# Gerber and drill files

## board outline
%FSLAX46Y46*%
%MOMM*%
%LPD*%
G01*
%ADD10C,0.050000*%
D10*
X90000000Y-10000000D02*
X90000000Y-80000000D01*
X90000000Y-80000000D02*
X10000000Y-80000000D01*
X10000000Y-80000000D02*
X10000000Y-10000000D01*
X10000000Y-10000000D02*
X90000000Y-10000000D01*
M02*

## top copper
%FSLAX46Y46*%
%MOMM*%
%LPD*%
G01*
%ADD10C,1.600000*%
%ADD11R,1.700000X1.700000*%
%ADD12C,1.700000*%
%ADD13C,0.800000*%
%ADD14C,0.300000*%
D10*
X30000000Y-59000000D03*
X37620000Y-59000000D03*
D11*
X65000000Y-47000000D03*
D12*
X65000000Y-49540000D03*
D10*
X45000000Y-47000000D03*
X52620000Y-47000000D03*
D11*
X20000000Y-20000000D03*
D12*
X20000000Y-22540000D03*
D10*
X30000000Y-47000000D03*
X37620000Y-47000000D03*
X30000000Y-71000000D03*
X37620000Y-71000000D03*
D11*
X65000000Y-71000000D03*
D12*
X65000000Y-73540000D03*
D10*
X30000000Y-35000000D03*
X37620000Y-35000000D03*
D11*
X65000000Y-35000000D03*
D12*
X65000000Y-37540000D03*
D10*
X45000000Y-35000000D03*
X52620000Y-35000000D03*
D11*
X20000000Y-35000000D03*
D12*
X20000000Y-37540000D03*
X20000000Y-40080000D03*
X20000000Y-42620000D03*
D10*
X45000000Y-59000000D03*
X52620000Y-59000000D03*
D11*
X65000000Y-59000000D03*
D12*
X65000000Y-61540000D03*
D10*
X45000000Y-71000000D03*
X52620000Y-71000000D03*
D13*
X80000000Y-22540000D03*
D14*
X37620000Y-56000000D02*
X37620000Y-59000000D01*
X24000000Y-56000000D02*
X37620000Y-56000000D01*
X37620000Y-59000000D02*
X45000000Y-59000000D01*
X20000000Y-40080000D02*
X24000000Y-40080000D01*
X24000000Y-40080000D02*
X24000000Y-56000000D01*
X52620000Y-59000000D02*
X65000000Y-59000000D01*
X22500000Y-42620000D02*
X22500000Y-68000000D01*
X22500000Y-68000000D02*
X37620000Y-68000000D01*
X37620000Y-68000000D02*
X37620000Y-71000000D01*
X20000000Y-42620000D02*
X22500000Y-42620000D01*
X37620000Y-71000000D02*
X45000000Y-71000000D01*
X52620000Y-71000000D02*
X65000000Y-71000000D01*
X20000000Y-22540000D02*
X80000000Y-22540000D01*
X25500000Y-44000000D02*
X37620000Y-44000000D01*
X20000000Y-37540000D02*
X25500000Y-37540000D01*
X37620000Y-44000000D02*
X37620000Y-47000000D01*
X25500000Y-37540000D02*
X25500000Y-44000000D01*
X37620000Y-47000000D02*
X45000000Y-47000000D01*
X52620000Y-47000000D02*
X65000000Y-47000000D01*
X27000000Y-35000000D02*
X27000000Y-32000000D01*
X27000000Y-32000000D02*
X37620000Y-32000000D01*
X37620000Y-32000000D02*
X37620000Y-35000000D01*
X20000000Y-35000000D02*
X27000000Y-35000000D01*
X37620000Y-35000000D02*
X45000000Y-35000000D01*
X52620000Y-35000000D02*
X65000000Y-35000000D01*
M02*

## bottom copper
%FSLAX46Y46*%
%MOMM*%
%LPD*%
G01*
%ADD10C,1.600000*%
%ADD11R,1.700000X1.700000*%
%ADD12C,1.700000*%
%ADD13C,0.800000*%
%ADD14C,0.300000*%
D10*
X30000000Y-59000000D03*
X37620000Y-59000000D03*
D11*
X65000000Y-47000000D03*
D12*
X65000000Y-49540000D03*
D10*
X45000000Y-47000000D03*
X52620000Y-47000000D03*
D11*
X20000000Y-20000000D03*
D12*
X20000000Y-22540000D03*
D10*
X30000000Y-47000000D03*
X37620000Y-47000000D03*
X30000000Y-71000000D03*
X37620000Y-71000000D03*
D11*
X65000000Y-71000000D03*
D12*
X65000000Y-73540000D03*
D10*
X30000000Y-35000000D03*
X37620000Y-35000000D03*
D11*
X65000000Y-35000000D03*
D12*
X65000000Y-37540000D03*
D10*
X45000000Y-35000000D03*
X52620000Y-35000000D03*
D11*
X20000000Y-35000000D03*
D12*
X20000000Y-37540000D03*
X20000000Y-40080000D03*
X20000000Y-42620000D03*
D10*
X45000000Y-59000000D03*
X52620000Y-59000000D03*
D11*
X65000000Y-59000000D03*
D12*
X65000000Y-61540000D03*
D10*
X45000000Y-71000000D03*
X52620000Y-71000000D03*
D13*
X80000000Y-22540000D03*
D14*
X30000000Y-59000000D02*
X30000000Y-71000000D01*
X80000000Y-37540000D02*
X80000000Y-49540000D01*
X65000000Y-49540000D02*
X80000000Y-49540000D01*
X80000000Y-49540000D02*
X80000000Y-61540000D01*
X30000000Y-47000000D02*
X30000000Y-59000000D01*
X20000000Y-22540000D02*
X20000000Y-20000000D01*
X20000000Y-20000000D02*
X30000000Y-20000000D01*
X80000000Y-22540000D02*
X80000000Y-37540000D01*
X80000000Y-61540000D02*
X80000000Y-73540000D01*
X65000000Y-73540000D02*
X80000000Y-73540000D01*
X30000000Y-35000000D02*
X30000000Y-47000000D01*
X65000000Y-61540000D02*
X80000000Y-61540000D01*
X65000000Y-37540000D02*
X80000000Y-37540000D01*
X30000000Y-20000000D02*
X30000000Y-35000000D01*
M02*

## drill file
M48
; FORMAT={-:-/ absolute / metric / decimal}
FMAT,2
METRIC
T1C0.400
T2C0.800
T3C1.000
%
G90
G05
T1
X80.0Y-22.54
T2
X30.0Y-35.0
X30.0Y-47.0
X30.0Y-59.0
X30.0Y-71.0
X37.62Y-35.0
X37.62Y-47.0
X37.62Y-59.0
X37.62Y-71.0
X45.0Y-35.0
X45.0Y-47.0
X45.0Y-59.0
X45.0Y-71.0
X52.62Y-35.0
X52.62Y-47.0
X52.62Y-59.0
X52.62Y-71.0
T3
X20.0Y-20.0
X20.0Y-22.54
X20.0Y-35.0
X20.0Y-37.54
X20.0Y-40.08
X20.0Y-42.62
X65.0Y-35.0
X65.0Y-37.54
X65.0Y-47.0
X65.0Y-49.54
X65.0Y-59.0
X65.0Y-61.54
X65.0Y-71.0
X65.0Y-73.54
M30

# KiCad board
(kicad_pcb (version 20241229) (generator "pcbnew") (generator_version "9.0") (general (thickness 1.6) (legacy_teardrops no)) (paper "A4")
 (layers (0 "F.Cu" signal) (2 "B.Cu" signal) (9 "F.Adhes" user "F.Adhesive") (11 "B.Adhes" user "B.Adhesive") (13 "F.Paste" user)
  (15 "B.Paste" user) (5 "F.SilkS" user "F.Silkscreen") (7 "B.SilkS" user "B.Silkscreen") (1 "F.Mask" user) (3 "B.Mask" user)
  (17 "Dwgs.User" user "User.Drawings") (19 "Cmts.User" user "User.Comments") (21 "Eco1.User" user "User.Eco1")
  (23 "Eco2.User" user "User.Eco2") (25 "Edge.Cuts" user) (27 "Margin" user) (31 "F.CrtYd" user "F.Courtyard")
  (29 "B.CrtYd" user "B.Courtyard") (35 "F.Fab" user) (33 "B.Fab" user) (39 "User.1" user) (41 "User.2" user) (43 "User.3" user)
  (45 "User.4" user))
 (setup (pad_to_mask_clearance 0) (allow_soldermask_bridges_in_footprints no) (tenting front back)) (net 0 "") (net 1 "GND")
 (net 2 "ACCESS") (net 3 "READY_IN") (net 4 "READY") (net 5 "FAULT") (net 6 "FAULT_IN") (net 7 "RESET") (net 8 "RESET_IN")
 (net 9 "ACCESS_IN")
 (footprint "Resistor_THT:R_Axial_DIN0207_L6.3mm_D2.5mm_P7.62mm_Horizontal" (layer "F.Cu") (at 30 59)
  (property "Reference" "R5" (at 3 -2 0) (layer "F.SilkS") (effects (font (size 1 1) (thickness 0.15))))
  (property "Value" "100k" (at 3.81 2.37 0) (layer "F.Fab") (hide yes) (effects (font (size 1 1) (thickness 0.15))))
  (pad "1" thru_hole circle (at 0 0) (size 1.6 1.6) (drill 0.8) (layers "*.Cu" "*.Mask") (remove_unused_layers no) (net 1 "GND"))
  (pad "2" thru_hole circle (at 7.62 0) (size 1.6 1.6) (drill 0.8) (layers "*.Cu" "*.Mask") (remove_unused_layers no) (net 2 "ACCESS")))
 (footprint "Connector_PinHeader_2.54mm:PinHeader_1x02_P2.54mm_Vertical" (layer "F.Cu") (at 65 47)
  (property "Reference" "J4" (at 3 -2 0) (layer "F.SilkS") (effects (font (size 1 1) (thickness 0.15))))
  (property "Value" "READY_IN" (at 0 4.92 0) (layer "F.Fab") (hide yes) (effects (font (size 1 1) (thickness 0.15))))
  (pad "1" thru_hole rect (at 0 0) (size 1.7 1.7) (drill 1) (layers "*.Cu" "*.Mask") (remove_unused_layers no) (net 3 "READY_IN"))
  (pad "2" thru_hole circle (at 0 2.54) (size 1.7 1.7) (drill 1) (layers "*.Cu" "*.Mask") (remove_unused_layers no) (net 1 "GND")))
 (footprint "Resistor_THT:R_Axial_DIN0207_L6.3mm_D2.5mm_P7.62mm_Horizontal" (layer "F.Cu") (at 45 47)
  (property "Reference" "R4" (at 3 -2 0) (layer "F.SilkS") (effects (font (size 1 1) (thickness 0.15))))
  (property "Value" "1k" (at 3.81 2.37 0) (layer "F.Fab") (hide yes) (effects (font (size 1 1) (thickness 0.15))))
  (pad "1" thru_hole circle (at 0 0) (size 1.6 1.6) (drill 0.8) (layers "*.Cu" "*.Mask") (remove_unused_layers no) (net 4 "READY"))
  (pad "2" thru_hole circle (at 7.62 0) (size 1.6 1.6) (drill 0.8) (layers "*.Cu" "*.Mask") (remove_unused_layers no) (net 3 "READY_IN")))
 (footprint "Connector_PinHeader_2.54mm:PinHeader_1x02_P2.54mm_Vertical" (layer "F.Cu") (at 20 20)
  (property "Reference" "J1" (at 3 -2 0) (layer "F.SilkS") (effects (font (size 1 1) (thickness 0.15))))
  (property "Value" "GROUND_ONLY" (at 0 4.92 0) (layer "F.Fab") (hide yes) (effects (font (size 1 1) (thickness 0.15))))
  (pad "1" thru_hole rect (at 0 0) (size 1.7 1.7) (drill 1) (layers "*.Cu" "*.Mask") (remove_unused_layers no) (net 1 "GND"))
  (pad "2" thru_hole circle (at 0 2.54) (size 1.7 1.7) (drill 1) (layers "*.Cu" "*.Mask") (remove_unused_layers no) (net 1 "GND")))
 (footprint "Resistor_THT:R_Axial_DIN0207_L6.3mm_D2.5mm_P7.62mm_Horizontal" (layer "F.Cu") (at 30 47)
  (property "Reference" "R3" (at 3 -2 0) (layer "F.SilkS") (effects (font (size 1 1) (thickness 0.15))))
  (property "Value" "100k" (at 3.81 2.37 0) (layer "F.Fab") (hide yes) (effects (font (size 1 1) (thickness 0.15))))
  (pad "1" thru_hole circle (at 0 0) (size 1.6 1.6) (drill 0.8) (layers "*.Cu" "*.Mask") (remove_unused_layers no) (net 1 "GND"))
  (pad "2" thru_hole circle (at 7.62 0) (size 1.6 1.6) (drill 0.8) (layers "*.Cu" "*.Mask") (remove_unused_layers no) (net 4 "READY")))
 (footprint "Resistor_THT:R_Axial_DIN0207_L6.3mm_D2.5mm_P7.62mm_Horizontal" (layer "F.Cu") (at 30 71)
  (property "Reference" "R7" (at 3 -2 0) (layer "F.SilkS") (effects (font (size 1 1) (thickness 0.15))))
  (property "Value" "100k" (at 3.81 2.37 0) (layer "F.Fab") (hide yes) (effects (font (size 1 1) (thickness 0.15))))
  (pad "1" thru_hole circle (at 0 0) (size 1.6 1.6) (drill 0.8) (layers "*.Cu" "*.Mask") (remove_unused_layers no) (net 1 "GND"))
  (pad "2" thru_hole circle (at 7.62 0) (size 1.6 1.6) (drill 0.8) (layers "*.Cu" "*.Mask") (remove_unused_layers no) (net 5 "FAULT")))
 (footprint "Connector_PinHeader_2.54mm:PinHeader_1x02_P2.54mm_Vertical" (layer "F.Cu") (at 65 71)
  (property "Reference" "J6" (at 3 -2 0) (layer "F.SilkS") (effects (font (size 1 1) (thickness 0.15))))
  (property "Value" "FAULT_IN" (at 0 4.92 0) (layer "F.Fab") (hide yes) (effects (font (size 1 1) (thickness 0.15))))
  (pad "1" thru_hole rect (at 0 0) (size 1.7 1.7) (drill 1) (layers "*.Cu" "*.Mask") (remove_unused_layers no) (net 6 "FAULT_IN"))
  (pad "2" thru_hole circle (at 0 2.54) (size 1.7 1.7) (drill 1) (layers "*.Cu" "*.Mask") (remove_unused_layers no) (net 1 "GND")))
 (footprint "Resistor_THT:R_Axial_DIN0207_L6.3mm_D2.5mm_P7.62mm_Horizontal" (layer "F.Cu") (at 30 35)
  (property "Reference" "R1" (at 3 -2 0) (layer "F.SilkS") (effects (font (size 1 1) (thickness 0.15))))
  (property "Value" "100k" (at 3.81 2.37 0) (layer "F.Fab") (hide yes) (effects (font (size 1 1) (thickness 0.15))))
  (pad "1" thru_hole circle (at 0 0) (size 1.6 1.6) (drill 0.8) (layers "*.Cu" "*.Mask") (remove_unused_layers no) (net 1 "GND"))
  (pad "2" thru_hole circle (at 7.62 0) (size 1.6 1.6) (drill 0.8) (layers "*.Cu" "*.Mask") (remove_unused_layers no) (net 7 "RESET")))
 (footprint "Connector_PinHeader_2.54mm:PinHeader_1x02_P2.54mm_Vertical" (layer "F.Cu") (at 65 35)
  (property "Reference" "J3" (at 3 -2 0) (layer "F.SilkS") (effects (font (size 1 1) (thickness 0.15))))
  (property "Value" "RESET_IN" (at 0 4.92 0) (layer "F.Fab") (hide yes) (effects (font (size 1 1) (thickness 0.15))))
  (pad "1" thru_hole rect (at 0 0) (size 1.7 1.7) (drill 1) (layers "*.Cu" "*.Mask") (remove_unused_layers no) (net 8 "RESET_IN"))
  (pad "2" thru_hole circle (at 0 2.54) (size 1.7 1.7) (drill 1) (layers "*.Cu" "*.Mask") (remove_unused_layers no) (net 1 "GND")))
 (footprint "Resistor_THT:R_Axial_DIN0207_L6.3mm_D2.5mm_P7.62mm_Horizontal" (layer "F.Cu") (at 45 35)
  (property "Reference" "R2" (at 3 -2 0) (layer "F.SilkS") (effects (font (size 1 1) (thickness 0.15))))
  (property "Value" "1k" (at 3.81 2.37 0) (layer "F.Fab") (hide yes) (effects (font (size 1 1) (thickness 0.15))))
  (pad "1" thru_hole circle (at 0 0) (size 1.6 1.6) (drill 0.8) (layers "*.Cu" "*.Mask") (remove_unused_layers no) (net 7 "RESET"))
  (pad "2" thru_hole circle (at 7.62 0) (size 1.6 1.6) (drill 0.8) (layers "*.Cu" "*.Mask") (remove_unused_layers no) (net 8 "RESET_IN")))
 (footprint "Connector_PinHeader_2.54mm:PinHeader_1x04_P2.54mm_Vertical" (layer "F.Cu") (at 20 35)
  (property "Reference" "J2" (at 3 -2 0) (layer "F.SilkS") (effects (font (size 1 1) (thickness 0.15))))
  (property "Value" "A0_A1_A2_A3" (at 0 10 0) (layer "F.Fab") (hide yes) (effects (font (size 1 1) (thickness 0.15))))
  (pad "1" thru_hole rect (at 0 0) (size 1.7 1.7) (drill 1) (layers "*.Cu" "*.Mask") (remove_unused_layers no) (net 7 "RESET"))
  (pad "2" thru_hole circle (at 0 2.54) (size 1.7 1.7) (drill 1) (layers "*.Cu" "*.Mask") (remove_unused_layers no) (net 4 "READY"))
  (pad "3" thru_hole circle (at 0 5.08) (size 1.7 1.7) (drill 1) (layers "*.Cu" "*.Mask") (remove_unused_layers no) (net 2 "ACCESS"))
  (pad "4" thru_hole circle (at 0 7.62) (size 1.7 1.7) (drill 1) (layers "*.Cu" "*.Mask") (remove_unused_layers no) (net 5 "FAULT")))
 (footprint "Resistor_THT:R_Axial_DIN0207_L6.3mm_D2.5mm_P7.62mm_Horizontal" (layer "F.Cu") (at 45 59)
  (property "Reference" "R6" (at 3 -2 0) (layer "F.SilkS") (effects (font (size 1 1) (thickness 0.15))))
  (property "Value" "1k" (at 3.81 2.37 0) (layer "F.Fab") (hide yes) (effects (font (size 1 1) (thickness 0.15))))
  (pad "1" thru_hole circle (at 0 0) (size 1.6 1.6) (drill 0.8) (layers "*.Cu" "*.Mask") (remove_unused_layers no) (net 2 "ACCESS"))
  (pad "2" thru_hole circle (at 7.62 0) (size 1.6 1.6) (drill 0.8) (layers "*.Cu" "*.Mask") (remove_unused_layers no) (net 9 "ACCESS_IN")))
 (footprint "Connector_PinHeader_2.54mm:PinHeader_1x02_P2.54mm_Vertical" (layer "F.Cu") (at 65 59)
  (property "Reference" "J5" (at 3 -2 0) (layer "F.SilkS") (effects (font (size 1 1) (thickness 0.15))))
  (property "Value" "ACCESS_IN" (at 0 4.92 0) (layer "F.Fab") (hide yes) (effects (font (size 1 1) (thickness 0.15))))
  (pad "1" thru_hole rect (at 0 0) (size 1.7 1.7) (drill 1) (layers "*.Cu" "*.Mask") (remove_unused_layers no) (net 9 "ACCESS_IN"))
  (pad "2" thru_hole circle (at 0 2.54) (size 1.7 1.7) (drill 1) (layers "*.Cu" "*.Mask") (remove_unused_layers no) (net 1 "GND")))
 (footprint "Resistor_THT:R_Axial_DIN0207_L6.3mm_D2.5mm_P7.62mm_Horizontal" (layer "F.Cu") (at 45 71)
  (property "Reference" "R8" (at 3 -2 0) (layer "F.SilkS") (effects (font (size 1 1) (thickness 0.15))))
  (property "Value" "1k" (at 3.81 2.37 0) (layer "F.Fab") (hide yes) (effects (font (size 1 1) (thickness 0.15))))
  (pad "1" thru_hole circle (at 0 0) (size 1.6 1.6) (drill 0.8) (layers "*.Cu" "*.Mask") (remove_unused_layers no) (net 5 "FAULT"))
  (pad "2" thru_hole circle (at 7.62 0) (size 1.6 1.6) (drill 0.8) (layers "*.Cu" "*.Mask") (remove_unused_layers no) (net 6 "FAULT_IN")))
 (gr_line (start 90 10) (end 90 80) (stroke (width 0.05) (type default)) (layer "Edge.Cuts"))
 (gr_line (start 90 80) (end 10 80) (stroke (width 0.05) (type default)) (layer "Edge.Cuts"))
 (gr_line (start 10 80) (end 10 10) (stroke (width 0.05) (type default)) (layer "Edge.Cuts"))
 (gr_line (start 10 10) (end 90 10) (stroke (width 0.05) (type default)) (layer "Edge.Cuts"))
 (segment (start 37.62 56) (end 37.62 59) (width 0.3) (layer "F.Cu") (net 2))
 (segment (start 24 56) (end 37.62 56) (width 0.3) (layer "F.Cu") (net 2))
 (segment (start 37.62 59) (end 45 59) (width 0.3) (layer "F.Cu") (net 2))
 (segment (start 20 40.08) (end 24 40.08) (width 0.3) (layer "F.Cu") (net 2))
 (segment (start 24 40.08) (end 24 56) (width 0.3) (layer "F.Cu") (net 2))
 (segment (start 52.62 59) (end 65 59) (width 0.3) (layer "F.Cu") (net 9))
 (segment (start 22.5 42.62) (end 22.5 68) (width 0.3) (layer "F.Cu") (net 5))
 (segment (start 22.5 68) (end 37.62 68) (width 0.3) (layer "F.Cu") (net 5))
 (segment (start 37.62 68) (end 37.62 71) (width 0.3) (layer "F.Cu") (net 5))
 (segment (start 20 42.62) (end 22.5 42.62) (width 0.3) (layer "F.Cu") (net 5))
 (segment (start 37.62 71) (end 45 71) (width 0.3) (layer "F.Cu") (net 5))
 (segment (start 52.62 71) (end 65 71) (width 0.3) (layer "F.Cu") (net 6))
 (segment (start 20 22.54) (end 80 22.54) (width 0.3) (layer "F.Cu") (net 1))
 (via (at 80 22.54) (size 0.8) (drill 0.4) (layers "F.Cu" "B.Cu") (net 1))
 (segment (start 30 59) (end 30 71) (width 0.3) (layer "B.Cu") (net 1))
 (segment (start 80 37.54) (end 80 49.54) (width 0.3) (layer "B.Cu") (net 1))
 (segment (start 65 49.54) (end 80 49.54) (width 0.3) (layer "B.Cu") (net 1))
 (segment (start 80 49.54) (end 80 61.54) (width 0.3) (layer "B.Cu") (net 1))
 (segment (start 30 47) (end 30 59) (width 0.3) (layer "B.Cu") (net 1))
 (segment (start 20 22.54) (end 20 20) (width 0.3) (layer "B.Cu") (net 1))
 (segment (start 20 20) (end 30 20) (width 0.3) (layer "B.Cu") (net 1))
 (segment (start 80 22.54) (end 80 37.54) (width 0.3) (layer "B.Cu") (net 1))
 (segment (start 80 61.54) (end 80 73.54) (width 0.3) (layer "B.Cu") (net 1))
 (segment (start 65 73.54) (end 80 73.54) (width 0.3) (layer "B.Cu") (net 1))
 (segment (start 30 35) (end 30 47) (width 0.3) (layer "B.Cu") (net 1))
 (segment (start 65 61.54) (end 80 61.54) (width 0.3) (layer "B.Cu") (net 1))
 (segment (start 65 37.54) (end 80 37.54) (width 0.3) (layer "B.Cu") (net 1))
 (segment (start 30 20) (end 30 35) (width 0.3) (layer "B.Cu") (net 1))
 (segment (start 25.5 44) (end 37.62 44) (width 0.3) (layer "F.Cu") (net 4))
 (segment (start 20 37.54) (end 25.5 37.54) (width 0.3) (layer "F.Cu") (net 4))
 (segment (start 37.62 44) (end 37.62 47) (width 0.3) (layer "F.Cu") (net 4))
 (segment (start 25.5 37.54) (end 25.5 44) (width 0.3) (layer "F.Cu") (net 4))
 (segment (start 37.62 47) (end 45 47) (width 0.3) (layer "F.Cu") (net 4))
 (segment (start 52.62 47) (end 65 47) (width 0.3) (layer "F.Cu") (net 3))
 (segment (start 27 35) (end 27 32) (width 0.3) (layer "F.Cu") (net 7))
 (segment (start 27 32) (end 37.62 32) (width 0.3) (layer "F.Cu") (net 7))
 (segment (start 37.62 32) (end 37.62 35) (width 0.3) (layer "F.Cu") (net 7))
 (segment (start 20 35) (end 27 35) (width 0.3) (layer "F.Cu") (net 7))
 (segment (start 37.62 35) (end 45 35) (width 0.3) (layer "F.Cu") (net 7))
 (segment (start 52.62 35) (end 65 35) (width 0.3) (layer "F.Cu") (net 8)))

